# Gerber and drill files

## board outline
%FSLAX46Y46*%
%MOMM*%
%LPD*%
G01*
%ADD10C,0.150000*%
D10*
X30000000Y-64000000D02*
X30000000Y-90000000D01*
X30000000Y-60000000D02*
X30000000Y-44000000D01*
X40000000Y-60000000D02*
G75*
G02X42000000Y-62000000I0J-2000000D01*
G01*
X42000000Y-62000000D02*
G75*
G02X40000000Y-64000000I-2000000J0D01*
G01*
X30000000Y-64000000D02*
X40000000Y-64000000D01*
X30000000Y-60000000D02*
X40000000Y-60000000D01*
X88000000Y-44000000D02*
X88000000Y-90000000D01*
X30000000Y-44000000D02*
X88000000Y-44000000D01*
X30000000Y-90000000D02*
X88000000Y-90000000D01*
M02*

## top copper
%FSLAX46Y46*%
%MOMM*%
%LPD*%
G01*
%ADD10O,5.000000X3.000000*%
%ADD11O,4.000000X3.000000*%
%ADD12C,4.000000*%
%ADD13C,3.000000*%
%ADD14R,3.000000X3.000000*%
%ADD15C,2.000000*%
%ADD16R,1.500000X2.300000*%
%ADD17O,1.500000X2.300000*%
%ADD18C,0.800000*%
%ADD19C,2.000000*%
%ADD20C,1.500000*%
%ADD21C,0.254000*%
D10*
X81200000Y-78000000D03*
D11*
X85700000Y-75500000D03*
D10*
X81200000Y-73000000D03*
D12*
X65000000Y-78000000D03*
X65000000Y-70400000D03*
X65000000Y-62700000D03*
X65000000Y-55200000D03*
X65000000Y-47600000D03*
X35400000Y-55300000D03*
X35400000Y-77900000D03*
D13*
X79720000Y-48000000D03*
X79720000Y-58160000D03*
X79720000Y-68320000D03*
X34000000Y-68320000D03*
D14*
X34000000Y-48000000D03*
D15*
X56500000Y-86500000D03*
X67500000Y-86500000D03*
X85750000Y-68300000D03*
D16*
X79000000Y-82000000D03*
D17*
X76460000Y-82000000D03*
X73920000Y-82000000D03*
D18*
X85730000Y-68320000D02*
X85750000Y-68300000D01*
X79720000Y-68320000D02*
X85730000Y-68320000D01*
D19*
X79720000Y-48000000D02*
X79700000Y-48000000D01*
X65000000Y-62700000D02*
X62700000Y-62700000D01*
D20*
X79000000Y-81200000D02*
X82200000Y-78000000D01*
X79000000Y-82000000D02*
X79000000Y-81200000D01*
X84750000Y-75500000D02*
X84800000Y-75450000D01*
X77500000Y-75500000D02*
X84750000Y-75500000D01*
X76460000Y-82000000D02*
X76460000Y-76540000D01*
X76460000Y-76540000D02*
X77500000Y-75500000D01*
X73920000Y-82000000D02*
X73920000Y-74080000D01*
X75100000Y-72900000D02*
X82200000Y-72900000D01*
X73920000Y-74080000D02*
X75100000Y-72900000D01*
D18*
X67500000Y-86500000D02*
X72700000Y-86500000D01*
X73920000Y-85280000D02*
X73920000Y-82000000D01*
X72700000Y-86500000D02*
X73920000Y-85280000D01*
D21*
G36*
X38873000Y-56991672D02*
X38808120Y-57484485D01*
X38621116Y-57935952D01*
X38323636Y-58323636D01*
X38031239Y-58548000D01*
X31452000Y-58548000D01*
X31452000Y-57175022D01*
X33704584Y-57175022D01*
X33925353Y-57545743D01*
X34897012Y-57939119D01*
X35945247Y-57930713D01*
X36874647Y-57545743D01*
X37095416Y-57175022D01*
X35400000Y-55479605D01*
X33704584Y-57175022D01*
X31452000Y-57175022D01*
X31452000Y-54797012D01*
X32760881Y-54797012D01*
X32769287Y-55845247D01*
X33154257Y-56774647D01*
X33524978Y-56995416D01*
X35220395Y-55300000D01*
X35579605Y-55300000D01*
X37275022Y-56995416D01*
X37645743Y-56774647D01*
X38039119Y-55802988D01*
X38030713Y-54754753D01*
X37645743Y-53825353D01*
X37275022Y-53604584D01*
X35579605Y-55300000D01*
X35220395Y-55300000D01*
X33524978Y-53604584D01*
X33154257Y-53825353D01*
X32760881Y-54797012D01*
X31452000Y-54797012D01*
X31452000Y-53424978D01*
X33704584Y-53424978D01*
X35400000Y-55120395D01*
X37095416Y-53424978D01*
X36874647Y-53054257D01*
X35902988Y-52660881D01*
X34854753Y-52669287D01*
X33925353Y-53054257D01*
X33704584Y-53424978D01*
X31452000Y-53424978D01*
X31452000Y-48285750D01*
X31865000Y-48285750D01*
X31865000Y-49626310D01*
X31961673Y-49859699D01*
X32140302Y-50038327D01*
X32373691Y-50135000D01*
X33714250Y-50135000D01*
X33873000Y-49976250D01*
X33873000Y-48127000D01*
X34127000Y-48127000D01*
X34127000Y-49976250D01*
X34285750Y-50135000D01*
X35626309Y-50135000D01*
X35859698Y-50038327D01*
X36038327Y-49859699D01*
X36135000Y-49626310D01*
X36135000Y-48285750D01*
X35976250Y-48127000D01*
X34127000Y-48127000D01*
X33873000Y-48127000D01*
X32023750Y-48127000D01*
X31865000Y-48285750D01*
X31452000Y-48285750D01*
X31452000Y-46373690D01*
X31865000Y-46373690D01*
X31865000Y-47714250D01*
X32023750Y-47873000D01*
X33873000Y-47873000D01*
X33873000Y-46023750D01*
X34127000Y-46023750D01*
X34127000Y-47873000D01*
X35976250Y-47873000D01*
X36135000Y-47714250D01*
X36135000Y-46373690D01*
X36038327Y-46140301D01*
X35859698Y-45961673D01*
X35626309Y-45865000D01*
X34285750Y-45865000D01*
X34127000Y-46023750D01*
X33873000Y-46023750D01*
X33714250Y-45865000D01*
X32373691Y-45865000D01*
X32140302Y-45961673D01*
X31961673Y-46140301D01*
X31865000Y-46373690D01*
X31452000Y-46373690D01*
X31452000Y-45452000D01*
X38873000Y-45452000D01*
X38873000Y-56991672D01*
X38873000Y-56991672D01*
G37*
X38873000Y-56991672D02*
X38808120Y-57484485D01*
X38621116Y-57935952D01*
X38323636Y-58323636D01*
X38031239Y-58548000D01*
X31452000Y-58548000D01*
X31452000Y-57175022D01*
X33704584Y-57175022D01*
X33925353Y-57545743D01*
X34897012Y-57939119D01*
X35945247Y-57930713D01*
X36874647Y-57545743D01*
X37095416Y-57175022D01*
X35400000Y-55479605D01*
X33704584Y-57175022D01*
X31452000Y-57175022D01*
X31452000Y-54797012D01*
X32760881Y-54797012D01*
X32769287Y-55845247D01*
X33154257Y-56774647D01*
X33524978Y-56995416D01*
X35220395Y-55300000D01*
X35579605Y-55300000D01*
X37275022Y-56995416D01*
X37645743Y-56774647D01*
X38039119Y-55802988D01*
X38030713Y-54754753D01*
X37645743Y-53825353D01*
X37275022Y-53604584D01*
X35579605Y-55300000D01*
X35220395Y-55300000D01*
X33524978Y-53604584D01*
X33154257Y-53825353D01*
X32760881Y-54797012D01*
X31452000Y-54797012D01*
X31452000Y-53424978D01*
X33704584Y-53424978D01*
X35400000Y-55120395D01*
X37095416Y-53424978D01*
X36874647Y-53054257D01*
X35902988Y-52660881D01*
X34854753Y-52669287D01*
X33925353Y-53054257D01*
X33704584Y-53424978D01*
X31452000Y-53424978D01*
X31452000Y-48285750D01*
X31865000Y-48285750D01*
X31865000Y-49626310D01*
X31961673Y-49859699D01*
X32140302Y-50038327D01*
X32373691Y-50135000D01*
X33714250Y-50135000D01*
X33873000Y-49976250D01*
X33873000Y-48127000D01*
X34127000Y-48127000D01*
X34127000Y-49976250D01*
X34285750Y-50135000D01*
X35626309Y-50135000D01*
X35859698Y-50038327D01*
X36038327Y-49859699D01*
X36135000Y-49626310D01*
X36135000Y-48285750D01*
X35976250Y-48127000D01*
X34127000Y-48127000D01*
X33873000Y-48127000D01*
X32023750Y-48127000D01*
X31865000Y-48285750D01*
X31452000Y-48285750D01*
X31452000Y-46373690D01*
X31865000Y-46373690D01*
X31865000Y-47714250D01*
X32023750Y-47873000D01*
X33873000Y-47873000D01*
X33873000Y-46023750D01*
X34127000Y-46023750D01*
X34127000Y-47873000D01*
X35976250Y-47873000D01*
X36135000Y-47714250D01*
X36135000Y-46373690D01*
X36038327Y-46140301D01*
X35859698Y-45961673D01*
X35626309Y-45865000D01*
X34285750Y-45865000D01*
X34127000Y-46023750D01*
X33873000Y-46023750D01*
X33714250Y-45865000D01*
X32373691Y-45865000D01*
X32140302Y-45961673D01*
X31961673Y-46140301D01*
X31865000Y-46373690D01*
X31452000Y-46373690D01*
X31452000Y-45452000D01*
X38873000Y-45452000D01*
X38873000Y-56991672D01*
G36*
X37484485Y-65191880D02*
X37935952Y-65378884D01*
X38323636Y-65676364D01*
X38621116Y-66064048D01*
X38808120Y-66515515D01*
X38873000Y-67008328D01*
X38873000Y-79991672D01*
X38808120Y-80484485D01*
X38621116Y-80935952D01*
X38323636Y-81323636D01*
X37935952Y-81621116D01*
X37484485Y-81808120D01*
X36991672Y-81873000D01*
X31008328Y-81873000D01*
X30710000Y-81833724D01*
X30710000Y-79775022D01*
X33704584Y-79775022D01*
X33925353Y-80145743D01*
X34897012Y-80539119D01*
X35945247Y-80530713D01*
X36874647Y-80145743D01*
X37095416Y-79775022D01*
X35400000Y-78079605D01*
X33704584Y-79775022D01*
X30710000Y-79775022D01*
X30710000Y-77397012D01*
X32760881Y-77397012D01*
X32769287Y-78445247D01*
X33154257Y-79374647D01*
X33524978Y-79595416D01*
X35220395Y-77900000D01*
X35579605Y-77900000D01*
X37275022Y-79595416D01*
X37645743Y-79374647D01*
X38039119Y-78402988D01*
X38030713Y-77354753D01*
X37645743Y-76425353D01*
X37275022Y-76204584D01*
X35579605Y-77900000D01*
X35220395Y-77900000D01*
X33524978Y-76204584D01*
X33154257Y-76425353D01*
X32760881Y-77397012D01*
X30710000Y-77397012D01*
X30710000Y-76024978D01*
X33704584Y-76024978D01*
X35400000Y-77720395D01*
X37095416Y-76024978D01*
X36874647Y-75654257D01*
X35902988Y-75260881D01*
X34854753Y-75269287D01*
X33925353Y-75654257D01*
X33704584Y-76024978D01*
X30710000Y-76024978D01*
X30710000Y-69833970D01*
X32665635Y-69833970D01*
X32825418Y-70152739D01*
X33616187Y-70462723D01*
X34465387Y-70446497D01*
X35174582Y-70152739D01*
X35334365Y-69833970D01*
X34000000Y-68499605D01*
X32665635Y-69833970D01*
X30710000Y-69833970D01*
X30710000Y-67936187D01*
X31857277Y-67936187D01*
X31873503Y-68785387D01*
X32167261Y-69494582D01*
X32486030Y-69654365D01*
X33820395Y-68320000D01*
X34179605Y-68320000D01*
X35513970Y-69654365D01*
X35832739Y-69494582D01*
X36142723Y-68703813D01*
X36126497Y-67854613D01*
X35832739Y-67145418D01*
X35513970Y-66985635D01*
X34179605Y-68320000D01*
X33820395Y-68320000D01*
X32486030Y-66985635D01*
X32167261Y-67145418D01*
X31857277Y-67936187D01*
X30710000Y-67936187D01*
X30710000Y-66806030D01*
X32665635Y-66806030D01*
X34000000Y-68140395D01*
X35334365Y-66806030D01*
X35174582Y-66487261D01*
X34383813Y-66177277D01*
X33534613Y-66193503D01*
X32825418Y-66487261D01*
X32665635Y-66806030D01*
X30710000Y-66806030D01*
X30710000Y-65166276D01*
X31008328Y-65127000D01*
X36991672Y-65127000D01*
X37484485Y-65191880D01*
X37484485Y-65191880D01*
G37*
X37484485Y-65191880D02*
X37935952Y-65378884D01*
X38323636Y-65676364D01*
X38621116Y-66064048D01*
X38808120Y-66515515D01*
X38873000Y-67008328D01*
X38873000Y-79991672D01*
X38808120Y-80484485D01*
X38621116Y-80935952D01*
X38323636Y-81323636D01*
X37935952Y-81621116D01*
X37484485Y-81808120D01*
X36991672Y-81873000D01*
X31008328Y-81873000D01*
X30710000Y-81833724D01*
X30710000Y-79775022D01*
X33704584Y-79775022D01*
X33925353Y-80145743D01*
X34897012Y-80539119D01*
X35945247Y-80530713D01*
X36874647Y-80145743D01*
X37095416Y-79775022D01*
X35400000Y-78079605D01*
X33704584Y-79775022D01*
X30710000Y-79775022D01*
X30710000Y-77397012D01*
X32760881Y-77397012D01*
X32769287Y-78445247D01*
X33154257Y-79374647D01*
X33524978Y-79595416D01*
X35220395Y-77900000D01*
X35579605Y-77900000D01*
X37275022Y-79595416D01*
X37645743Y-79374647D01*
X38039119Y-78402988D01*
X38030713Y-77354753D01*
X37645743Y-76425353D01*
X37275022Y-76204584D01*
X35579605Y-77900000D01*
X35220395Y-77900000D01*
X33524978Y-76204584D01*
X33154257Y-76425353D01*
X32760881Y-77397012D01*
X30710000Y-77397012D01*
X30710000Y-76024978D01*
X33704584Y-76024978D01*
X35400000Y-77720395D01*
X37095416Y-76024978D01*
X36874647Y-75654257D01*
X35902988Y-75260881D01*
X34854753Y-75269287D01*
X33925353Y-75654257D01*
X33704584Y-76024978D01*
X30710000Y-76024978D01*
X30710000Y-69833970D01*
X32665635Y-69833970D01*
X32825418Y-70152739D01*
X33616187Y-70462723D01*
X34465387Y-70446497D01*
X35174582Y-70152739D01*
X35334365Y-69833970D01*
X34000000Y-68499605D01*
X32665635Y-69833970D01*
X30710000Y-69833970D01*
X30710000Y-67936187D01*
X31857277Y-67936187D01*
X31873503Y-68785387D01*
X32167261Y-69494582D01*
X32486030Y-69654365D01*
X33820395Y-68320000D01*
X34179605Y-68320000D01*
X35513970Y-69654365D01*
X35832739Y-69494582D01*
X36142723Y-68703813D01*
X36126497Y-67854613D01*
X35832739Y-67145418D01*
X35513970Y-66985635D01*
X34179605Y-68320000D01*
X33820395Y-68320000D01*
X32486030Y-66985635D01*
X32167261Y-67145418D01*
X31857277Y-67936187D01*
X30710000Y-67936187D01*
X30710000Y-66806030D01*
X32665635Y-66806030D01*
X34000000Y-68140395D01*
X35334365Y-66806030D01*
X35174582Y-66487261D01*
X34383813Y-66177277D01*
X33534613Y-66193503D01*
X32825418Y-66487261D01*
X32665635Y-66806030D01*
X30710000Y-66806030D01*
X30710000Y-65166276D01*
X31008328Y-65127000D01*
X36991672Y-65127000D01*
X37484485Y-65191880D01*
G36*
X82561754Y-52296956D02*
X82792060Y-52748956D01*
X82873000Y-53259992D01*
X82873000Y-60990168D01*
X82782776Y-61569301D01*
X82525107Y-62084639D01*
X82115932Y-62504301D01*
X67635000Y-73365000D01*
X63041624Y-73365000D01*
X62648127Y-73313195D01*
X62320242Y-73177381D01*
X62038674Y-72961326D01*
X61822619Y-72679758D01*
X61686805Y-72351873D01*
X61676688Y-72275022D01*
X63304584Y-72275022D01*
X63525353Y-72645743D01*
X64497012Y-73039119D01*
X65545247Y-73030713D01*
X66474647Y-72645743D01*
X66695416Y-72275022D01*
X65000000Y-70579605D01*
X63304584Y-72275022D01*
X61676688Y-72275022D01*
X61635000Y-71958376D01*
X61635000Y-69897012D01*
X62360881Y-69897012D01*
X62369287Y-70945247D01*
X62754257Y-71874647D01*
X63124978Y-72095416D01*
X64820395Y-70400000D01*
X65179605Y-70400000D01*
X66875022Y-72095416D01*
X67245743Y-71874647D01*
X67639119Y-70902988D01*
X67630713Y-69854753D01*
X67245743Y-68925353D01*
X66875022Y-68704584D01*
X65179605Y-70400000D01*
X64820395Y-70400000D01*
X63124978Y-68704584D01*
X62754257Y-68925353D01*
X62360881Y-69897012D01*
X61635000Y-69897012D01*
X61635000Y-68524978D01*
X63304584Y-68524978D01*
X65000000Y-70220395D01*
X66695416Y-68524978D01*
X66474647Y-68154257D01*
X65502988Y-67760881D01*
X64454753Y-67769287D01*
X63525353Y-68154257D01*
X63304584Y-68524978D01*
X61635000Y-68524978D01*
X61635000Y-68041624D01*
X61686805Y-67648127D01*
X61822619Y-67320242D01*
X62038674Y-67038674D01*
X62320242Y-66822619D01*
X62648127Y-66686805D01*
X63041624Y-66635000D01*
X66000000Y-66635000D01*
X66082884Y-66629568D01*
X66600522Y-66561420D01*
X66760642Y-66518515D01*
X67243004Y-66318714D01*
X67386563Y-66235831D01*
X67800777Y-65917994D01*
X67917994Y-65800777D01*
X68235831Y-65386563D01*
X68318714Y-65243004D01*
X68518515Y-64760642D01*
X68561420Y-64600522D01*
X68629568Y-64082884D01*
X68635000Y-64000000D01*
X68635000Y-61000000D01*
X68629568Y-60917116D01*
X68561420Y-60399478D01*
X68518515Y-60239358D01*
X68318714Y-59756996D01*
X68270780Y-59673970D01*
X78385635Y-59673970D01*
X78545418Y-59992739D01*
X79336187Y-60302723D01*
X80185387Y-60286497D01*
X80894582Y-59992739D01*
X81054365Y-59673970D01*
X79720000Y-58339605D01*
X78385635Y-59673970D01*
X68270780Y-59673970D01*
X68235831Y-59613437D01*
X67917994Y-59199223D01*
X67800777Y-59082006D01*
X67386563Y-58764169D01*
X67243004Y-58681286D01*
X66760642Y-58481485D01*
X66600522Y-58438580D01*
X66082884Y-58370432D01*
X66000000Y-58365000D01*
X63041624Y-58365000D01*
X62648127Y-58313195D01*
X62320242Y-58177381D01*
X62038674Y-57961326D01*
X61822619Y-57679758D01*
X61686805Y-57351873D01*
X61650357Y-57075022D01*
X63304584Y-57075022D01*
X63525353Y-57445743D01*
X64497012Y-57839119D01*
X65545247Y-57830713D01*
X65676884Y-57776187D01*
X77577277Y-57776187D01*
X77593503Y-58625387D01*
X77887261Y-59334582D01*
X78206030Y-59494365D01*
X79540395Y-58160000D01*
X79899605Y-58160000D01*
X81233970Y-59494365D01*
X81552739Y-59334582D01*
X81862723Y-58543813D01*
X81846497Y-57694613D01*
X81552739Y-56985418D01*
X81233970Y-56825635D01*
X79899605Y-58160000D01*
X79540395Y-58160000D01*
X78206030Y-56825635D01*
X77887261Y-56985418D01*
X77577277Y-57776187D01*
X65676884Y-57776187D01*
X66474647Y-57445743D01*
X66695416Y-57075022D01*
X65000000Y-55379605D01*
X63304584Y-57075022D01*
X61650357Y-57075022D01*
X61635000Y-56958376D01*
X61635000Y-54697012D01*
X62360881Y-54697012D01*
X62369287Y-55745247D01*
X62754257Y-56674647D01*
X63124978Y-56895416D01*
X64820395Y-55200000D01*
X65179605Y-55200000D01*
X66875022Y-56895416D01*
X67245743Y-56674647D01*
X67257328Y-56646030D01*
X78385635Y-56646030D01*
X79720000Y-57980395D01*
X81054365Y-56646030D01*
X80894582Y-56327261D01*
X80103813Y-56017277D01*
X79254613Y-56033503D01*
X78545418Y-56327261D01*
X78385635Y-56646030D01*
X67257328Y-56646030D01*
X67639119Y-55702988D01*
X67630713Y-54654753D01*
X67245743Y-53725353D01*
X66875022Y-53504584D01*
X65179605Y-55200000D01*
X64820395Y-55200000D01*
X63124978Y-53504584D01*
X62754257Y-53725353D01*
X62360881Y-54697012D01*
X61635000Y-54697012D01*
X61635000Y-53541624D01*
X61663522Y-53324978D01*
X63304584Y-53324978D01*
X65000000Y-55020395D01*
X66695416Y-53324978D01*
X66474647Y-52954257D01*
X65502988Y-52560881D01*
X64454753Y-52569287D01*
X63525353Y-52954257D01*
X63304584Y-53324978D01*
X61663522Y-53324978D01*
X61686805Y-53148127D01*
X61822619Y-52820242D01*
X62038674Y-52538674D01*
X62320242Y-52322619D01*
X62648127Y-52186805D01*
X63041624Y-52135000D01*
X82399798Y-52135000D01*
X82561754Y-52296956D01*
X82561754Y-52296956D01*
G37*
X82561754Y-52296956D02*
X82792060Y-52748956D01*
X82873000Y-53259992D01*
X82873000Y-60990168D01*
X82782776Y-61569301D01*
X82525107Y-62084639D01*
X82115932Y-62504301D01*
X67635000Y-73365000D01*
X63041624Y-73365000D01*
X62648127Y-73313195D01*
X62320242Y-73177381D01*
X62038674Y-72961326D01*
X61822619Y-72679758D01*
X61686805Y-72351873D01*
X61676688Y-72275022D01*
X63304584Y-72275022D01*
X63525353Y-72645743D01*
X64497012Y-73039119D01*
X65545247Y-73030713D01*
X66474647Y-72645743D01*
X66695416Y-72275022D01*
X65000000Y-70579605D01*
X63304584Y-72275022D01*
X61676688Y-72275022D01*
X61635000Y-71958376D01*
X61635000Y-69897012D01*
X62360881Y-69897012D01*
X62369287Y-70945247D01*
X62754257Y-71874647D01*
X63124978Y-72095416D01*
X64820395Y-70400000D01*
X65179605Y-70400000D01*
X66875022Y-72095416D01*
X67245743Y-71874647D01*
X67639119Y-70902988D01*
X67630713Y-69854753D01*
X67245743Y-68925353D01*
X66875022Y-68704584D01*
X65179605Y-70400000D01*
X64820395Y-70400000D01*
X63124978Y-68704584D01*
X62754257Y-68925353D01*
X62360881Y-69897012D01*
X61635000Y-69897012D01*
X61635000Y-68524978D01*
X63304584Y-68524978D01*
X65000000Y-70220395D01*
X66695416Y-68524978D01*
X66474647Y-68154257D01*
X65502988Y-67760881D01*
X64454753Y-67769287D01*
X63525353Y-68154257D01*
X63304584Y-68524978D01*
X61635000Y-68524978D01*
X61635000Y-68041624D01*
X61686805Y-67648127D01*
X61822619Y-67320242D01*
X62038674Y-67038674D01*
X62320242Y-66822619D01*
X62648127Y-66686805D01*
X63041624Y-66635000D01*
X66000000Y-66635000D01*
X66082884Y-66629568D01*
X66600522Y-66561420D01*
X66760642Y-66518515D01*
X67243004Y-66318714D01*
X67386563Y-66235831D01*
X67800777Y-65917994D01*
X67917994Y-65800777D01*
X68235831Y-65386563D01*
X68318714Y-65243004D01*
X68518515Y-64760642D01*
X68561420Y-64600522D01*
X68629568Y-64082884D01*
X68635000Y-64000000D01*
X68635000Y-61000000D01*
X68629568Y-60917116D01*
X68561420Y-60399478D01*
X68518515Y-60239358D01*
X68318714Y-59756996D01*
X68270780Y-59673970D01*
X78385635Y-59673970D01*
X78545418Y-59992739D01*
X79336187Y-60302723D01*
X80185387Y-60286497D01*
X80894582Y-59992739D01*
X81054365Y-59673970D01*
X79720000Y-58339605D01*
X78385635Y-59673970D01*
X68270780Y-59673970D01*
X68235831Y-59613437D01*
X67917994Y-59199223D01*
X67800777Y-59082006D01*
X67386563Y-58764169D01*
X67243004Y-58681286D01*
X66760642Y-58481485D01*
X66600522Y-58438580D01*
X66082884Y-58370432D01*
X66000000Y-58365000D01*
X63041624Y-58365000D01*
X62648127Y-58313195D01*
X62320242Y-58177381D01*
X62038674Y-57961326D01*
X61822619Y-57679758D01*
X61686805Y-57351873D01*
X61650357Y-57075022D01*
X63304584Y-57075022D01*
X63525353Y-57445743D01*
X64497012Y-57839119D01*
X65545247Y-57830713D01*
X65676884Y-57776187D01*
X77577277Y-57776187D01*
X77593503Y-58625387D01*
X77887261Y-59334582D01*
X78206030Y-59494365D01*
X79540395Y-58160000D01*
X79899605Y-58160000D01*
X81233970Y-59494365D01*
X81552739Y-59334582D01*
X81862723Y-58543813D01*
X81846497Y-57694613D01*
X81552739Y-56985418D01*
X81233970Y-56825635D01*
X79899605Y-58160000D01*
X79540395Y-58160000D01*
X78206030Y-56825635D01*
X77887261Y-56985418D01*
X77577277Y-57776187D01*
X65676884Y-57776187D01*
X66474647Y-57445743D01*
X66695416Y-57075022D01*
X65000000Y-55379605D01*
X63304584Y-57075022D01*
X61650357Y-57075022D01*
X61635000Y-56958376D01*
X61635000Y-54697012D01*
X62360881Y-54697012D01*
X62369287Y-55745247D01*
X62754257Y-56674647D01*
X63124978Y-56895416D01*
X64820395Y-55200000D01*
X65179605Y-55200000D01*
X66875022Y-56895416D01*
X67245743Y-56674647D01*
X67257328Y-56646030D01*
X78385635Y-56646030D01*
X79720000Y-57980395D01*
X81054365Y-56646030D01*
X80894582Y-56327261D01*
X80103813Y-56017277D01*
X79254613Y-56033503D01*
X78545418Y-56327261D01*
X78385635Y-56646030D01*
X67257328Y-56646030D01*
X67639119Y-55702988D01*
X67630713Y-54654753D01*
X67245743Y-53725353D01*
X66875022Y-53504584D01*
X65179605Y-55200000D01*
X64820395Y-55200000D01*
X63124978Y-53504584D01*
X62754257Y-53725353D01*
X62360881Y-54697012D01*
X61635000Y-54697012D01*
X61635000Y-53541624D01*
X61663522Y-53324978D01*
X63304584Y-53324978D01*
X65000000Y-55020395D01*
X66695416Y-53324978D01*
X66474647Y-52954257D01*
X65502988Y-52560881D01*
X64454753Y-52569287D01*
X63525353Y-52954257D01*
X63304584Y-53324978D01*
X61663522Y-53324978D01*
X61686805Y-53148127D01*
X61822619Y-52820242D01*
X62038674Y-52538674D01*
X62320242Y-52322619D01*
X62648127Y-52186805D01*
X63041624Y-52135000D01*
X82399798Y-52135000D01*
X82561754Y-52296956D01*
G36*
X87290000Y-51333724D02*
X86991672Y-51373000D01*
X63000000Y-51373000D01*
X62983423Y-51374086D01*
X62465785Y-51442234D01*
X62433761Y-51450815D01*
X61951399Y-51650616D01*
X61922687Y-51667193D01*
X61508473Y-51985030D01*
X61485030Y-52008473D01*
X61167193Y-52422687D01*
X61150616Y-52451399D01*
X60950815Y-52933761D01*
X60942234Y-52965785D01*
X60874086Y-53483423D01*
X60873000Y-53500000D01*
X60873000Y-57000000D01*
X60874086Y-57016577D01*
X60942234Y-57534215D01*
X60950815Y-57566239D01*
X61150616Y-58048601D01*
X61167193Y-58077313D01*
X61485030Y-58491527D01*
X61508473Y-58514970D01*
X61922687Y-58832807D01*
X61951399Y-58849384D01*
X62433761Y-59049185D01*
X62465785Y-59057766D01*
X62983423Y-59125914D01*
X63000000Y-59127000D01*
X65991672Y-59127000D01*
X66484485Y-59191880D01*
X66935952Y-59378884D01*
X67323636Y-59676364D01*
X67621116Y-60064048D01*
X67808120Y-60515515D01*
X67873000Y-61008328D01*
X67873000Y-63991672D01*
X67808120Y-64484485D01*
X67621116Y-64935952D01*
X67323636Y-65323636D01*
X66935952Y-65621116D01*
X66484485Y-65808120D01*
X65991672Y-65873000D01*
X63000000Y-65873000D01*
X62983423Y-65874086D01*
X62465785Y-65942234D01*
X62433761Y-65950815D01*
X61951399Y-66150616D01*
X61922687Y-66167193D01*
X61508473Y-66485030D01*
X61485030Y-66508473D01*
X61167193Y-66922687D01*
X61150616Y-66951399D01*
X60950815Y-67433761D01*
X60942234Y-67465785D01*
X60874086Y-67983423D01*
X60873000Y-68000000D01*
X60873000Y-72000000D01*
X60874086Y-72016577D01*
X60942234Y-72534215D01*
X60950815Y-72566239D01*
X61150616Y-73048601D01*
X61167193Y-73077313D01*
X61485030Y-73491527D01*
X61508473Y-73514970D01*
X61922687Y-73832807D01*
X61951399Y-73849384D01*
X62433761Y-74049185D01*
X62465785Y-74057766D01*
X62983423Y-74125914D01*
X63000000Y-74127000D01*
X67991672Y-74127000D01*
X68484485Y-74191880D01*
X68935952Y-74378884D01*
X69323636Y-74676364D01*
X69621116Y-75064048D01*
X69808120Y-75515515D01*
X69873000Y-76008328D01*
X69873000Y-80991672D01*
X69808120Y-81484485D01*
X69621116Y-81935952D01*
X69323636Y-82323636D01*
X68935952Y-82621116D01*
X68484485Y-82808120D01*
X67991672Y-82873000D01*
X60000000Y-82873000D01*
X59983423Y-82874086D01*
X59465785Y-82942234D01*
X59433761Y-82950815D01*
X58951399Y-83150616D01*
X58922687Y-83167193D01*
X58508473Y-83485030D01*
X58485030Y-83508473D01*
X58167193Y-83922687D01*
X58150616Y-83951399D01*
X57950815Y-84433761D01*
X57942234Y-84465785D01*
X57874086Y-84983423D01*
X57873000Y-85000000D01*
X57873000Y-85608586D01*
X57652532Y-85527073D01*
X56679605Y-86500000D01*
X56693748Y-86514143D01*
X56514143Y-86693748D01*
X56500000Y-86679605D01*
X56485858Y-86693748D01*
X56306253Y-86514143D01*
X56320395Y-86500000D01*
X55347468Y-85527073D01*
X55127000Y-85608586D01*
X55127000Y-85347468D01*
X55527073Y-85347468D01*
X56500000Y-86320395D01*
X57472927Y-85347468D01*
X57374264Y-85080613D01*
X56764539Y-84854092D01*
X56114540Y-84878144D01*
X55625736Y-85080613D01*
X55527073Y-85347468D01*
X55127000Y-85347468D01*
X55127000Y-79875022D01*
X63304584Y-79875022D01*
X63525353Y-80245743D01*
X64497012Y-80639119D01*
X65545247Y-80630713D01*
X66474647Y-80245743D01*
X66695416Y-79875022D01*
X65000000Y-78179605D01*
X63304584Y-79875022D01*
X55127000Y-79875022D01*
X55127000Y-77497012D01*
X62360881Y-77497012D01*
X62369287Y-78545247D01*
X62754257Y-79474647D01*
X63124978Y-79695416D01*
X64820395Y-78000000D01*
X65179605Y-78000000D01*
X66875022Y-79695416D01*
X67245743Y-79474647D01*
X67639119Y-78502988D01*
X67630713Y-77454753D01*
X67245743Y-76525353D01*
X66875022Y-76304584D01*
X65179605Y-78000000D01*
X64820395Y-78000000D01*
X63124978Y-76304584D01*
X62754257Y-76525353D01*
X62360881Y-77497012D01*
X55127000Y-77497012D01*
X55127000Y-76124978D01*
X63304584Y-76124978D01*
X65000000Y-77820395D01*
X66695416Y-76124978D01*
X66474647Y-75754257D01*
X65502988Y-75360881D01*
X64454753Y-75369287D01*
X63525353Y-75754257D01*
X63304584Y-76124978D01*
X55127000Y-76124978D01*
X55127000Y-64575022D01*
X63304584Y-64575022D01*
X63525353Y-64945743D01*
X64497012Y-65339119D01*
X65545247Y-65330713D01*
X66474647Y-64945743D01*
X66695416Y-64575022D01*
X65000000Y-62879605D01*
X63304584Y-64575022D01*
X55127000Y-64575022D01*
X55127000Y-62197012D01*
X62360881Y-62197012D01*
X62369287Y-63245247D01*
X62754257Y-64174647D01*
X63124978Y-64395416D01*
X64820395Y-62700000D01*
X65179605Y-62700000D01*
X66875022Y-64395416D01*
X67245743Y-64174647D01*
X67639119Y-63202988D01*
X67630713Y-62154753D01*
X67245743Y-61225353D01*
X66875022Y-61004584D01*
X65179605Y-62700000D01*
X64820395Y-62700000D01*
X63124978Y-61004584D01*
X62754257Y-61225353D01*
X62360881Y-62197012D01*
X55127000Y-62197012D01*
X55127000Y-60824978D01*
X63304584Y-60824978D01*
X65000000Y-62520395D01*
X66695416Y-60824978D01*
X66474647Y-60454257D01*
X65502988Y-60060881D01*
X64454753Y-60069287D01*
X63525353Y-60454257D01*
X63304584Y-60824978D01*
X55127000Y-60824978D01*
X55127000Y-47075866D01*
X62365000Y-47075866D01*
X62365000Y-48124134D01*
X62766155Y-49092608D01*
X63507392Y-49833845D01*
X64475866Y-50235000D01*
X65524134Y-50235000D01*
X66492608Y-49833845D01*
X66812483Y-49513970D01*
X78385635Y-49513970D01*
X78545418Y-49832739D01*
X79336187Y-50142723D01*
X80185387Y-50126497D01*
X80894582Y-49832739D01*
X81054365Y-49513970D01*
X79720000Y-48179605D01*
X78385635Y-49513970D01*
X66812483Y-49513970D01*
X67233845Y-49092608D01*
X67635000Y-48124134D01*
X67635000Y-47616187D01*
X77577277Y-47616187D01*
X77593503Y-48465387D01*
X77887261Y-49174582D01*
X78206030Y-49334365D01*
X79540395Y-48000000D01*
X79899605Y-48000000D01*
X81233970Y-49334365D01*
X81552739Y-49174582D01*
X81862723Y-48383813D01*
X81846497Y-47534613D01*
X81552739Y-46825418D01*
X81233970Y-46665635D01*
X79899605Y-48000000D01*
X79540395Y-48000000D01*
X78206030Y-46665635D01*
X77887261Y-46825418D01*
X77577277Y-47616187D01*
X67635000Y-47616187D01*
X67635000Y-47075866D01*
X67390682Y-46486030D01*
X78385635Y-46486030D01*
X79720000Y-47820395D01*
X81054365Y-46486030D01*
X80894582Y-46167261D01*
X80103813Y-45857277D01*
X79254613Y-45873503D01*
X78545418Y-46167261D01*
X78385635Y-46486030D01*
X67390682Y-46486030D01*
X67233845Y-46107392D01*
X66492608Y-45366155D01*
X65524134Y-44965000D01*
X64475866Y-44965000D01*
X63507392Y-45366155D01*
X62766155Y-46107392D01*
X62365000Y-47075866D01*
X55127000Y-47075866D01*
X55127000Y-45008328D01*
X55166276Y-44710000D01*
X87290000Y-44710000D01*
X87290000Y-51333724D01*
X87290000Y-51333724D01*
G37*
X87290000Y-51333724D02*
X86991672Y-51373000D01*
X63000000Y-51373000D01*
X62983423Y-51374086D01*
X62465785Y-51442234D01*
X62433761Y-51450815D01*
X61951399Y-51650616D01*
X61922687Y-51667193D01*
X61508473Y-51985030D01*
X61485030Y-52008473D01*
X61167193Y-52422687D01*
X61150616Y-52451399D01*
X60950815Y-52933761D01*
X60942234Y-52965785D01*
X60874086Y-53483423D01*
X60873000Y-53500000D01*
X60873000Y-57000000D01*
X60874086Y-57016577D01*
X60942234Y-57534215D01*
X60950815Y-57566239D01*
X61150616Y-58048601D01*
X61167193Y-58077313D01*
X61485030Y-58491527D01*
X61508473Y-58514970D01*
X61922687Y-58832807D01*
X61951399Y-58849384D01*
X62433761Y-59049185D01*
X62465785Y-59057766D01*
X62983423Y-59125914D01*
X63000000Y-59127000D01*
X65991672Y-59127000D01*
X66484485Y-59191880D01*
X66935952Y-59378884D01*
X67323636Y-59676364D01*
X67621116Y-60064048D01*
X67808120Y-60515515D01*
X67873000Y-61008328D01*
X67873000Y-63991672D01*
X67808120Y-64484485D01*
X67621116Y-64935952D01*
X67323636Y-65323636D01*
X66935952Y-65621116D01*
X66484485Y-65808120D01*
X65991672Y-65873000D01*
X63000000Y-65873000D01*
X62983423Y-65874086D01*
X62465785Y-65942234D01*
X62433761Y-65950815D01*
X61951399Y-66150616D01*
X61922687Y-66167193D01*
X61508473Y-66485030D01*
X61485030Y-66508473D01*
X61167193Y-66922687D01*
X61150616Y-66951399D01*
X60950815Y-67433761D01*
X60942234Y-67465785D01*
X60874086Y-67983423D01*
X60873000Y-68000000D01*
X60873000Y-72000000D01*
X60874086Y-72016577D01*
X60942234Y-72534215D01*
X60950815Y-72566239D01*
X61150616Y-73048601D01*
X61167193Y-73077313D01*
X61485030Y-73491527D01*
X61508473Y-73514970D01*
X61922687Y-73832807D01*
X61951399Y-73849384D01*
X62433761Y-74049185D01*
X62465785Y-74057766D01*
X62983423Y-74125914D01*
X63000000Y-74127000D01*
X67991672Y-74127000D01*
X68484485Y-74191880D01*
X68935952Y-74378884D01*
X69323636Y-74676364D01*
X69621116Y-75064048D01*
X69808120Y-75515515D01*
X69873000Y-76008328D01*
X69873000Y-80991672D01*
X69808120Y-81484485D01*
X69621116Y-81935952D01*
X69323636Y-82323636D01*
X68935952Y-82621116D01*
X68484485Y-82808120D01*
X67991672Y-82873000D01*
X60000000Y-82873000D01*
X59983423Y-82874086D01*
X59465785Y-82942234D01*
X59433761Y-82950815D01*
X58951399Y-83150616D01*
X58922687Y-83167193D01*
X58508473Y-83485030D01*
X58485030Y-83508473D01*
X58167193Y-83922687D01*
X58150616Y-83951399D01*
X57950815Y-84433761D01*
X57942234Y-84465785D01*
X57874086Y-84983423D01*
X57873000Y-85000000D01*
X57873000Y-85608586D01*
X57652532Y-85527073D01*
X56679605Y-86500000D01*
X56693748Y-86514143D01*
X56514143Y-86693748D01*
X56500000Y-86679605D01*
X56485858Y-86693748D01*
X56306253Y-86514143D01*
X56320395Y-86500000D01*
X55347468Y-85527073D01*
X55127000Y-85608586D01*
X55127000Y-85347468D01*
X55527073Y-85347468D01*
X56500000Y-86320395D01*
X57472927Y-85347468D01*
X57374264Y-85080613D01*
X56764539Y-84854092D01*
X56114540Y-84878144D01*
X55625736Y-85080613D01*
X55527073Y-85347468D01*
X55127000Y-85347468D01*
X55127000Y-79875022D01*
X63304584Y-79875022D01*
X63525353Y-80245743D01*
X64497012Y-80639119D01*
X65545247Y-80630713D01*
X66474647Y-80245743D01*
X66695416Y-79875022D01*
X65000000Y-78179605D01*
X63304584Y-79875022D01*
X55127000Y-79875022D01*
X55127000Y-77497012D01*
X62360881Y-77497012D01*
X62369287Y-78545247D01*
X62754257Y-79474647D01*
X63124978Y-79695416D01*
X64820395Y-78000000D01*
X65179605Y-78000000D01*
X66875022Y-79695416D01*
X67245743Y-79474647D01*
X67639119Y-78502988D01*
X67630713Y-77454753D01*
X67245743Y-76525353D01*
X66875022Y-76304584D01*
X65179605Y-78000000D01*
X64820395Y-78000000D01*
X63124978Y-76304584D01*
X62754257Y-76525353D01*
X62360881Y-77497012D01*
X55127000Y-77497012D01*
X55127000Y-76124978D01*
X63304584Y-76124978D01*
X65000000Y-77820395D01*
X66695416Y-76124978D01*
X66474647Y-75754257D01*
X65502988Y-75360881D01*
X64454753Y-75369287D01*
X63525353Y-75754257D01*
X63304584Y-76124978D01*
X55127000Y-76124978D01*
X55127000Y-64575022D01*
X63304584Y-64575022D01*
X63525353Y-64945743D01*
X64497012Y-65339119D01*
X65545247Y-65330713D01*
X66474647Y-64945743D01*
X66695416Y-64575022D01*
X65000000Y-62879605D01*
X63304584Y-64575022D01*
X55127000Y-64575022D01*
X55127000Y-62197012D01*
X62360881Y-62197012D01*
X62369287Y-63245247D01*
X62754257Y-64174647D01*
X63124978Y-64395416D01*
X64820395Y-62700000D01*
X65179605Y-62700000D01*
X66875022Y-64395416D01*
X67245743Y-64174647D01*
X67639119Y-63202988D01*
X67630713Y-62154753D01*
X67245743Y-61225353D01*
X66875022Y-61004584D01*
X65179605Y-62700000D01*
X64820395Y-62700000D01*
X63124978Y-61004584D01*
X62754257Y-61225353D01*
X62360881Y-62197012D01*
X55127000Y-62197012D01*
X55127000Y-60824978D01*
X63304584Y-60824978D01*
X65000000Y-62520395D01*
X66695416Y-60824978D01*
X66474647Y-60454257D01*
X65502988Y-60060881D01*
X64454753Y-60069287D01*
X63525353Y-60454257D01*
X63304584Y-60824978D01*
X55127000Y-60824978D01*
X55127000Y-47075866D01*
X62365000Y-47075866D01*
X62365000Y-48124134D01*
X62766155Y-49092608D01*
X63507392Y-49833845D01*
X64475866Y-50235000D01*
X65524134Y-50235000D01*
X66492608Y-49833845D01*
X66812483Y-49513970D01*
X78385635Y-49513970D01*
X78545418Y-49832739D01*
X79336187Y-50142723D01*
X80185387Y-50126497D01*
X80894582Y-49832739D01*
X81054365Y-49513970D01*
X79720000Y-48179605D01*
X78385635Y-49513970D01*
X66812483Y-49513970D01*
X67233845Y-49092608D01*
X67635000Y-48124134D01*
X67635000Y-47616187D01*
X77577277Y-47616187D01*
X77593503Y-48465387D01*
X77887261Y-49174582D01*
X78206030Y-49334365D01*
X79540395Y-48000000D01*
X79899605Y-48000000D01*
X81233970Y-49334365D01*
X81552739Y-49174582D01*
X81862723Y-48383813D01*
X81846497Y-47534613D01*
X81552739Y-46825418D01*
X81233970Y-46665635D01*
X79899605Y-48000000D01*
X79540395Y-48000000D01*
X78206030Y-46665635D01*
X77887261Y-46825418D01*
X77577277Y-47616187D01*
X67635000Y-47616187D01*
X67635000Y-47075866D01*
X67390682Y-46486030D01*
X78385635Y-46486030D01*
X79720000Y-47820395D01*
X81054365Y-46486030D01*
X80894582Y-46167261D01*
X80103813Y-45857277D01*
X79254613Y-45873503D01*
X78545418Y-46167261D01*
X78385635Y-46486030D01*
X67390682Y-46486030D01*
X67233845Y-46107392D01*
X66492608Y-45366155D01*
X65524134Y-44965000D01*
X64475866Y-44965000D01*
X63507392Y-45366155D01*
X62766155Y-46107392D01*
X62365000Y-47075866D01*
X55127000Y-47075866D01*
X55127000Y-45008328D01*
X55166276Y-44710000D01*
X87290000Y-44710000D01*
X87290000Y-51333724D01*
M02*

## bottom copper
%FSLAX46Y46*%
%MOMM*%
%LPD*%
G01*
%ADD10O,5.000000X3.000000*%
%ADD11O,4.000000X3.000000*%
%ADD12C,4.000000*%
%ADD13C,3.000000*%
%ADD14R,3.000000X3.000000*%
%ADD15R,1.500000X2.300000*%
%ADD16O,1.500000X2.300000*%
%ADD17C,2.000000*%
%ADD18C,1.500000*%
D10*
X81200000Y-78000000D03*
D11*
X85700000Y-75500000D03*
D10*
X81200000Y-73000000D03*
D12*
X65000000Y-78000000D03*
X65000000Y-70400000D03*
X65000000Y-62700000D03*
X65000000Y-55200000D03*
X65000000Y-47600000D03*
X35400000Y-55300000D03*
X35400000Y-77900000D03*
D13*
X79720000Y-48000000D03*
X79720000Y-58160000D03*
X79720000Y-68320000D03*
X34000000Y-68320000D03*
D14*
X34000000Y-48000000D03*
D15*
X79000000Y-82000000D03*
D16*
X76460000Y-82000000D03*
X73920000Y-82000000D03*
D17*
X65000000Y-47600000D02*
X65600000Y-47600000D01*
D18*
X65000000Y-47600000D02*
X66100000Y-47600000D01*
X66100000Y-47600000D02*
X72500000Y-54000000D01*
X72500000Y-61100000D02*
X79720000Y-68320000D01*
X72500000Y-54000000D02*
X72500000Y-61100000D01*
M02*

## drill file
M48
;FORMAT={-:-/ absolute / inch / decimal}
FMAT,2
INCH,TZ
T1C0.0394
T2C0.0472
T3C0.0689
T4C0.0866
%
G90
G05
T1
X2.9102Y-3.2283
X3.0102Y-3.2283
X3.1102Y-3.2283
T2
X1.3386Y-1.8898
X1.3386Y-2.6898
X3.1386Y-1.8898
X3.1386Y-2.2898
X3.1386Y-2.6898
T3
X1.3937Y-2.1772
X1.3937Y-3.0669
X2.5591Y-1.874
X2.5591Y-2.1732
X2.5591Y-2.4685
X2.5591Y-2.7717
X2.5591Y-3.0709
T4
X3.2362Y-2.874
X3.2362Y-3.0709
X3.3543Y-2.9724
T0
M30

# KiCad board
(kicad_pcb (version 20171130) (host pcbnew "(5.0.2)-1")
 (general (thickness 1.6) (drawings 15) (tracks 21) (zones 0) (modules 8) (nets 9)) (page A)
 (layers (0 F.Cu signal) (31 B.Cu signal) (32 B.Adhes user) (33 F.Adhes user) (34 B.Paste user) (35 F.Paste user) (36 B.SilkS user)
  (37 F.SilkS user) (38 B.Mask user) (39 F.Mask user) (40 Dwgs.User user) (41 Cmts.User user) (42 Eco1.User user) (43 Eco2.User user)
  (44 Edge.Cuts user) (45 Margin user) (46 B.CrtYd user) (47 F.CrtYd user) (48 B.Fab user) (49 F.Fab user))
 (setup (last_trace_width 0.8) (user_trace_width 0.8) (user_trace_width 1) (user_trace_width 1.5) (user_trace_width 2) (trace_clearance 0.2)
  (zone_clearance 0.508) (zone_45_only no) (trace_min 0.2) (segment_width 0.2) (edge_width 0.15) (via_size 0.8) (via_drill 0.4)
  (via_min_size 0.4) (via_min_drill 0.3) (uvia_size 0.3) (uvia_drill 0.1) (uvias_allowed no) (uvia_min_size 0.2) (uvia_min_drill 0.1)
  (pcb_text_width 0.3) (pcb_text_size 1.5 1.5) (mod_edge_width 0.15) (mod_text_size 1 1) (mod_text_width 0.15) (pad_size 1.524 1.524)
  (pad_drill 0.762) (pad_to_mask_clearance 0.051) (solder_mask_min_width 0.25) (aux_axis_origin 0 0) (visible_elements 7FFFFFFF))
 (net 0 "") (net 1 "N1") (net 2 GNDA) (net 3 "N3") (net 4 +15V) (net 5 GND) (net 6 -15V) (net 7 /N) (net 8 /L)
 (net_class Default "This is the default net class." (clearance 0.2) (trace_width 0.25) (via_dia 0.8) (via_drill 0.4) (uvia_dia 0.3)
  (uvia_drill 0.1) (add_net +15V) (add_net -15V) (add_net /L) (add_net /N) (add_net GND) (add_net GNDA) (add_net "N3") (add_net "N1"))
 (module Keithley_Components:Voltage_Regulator (layer F.Cu) (at 82.2 78 270)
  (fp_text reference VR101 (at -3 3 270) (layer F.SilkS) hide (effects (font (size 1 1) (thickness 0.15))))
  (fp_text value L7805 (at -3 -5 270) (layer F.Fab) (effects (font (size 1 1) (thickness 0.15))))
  (pad 1 thru_hole oval (at 0 0 270) (size 3 5) (drill 2.2 (offset 0 1)) (layers *.Cu *.Mask) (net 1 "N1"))
  (pad 2 thru_hole oval (at -2.5 -3 270) (size 3 4) (drill 2.2 (offset 0 -0.5)) (layers *.Cu *.Mask) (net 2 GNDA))
  (pad 3 thru_hole oval (at -5 0 270) (size 3 5) (drill 2.2 (offset 0 1)) (layers *.Cu *.Mask) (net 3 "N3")))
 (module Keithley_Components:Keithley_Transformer (layer F.Cu) (at 65 83 180)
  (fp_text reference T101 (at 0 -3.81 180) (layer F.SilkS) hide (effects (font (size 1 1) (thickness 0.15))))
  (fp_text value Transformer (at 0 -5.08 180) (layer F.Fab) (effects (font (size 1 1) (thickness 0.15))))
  (pad 2 thru_hole circle (at 0 5 180) (size 4 4) (drill 1.75) (layers *.Cu *.Mask) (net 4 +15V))
  (pad 3 thru_hole circle (at 0 12.6 180) (size 4 4) (drill 1.75) (layers *.Cu *.Mask) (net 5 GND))
  (pad 4 thru_hole circle (at 0 20.3 180) (size 4 4) (drill 1.75) (layers *.Cu *.Mask) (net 4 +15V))
  (pad 5 thru_hole circle (at 0 27.8 180) (size 4 4) (drill 1.75) (layers *.Cu *.Mask) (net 5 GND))
  (pad 6 thru_hole circle (at 0 35.4 180) (size 4 4) (drill 1.75) (layers *.Cu *.Mask) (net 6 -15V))
  (pad 8 thru_hole circle (at 29.6 27.7 180) (size 4 4) (drill 1.75) (layers *.Cu *.Mask) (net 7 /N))
  (pad 11 thru_hole circle (at 29.6 5.1 180) (size 4 4) (drill 1.75) (layers *.Cu *.Mask) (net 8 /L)))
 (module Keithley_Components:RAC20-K (layer F.Cu) (at 34 48)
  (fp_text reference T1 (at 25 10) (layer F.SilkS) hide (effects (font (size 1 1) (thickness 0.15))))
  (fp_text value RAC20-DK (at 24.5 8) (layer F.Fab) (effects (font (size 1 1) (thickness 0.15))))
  (pad 5 thru_hole circle (at 45.72 0) (size 3 3) (drill 1.2) (layers *.Cu *.Mask) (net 4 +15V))
  (pad 4 thru_hole circle (at 45.72 10.16) (size 3 3) (drill 1.2) (layers *.Cu *.Mask) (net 5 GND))
  (pad 3 thru_hole circle (at 45.72 20.32) (size 3 3) (drill 1.2) (layers *.Cu *.Mask) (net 6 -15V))
  (pad 2 thru_hole circle (at 0 20.32) (size 3 3) (drill 1.2) (layers *.Cu *.Mask) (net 8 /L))
  (pad 1 thru_hole rect (at 0 0) (size 3 3) (drill 1.2) (layers *.Cu *.Mask) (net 7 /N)))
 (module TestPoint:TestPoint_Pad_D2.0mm (layer F.Cu) (at 56.5 86.5)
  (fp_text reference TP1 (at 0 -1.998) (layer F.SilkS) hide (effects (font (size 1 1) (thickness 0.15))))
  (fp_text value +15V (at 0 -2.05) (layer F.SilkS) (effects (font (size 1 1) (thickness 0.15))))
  (pad 1 smd circle (at 0 0) (size 2 2) (layers F.Cu F.Mask) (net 4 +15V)))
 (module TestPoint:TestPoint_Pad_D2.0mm (layer F.Cu) (at 67.5 86.5)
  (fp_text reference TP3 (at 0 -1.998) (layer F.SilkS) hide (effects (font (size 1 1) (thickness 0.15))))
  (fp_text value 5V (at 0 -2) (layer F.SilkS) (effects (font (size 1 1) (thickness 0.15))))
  (pad 1 smd circle (at 0 0) (size 2 2) (layers F.Cu F.Mask) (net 3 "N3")))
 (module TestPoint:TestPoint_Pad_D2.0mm (layer F.Cu) (at 85.75 68.3)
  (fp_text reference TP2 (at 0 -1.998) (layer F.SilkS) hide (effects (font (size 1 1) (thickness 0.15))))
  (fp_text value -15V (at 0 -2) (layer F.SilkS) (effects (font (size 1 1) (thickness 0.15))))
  (pad 1 smd circle (at 0 0) (size 2 2) (layers F.Cu F.Mask) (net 6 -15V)))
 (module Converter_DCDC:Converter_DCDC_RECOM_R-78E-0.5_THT (layer F.Cu) (at 79 82 180)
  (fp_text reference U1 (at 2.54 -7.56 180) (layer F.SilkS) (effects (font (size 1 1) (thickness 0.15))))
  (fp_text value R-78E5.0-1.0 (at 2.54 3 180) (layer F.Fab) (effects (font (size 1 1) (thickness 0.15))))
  (pad 1 thru_hole rect (at 0 0 180) (size 1.5 2.3) (drill 1) (layers *.Cu *.Mask) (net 1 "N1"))
  (pad 2 thru_hole oval (at 2.54 0 180) (size 1.5 2.3) (drill 1) (layers *.Cu *.Mask) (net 2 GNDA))
  (pad 3 thru_hole oval (at 5.08 0 180) (size 1.5 2.3) (drill 1) (layers *.Cu *.Mask) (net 3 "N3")))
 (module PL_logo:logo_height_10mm (layer F.Cu) (at 43.75 80)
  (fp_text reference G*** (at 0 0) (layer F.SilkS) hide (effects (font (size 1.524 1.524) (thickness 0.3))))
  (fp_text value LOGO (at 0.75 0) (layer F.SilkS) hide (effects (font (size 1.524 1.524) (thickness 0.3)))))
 (gr_line (start 30 64) (end 30 90) (layer Edge.Cuts) (width 0.15))
 (gr_line (start 30 60) (end 30 44) (layer Edge.Cuts) (width 0.15))
 (gr_arc (start 40 62) (end 42 62) (angle -90) (layer Edge.Cuts) (width 0.15))
 (gr_arc (start 40 62) (end 40 64) (angle -90) (layer Edge.Cuts) (width 0.15))
 (gr_line (start 30 64) (end 40 64) (layer Edge.Cuts) (width 0.15))
 (gr_line (start 30 60) (end 40 60) (layer Edge.Cuts) (width 0.15))
 (gr_line (start 88 44) (end 88 90) (layer Edge.Cuts) (width 0.15))
 (gr_line (start 30 44) (end 88 44) (layer Edge.Cuts) (width 0.15))
 (gr_line (start 30 90) (end 88 90) (layer Edge.Cuts) (width 0.15))
 (segment (start 65 47.6) (end 65.6 47.6) (width 2) (layer B.Cu) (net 6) (status 30))
 (segment (start 65 47.6) (end 66.1 47.6) (width 1.5) (layer B.Cu) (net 6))
 (segment (start 66.1 47.6) (end 72.5 54) (width 1.5) (layer B.Cu) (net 6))
 (segment (start 72.5 61.1) (end 79.72 68.32) (width 1.5) (layer B.Cu) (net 6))
 (segment (start 72.5 54) (end 72.5 61.1) (width 1.5) (layer B.Cu) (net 6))
 (segment (start 85.73 68.32) (end 85.75 68.3) (width 0.8) (layer F.Cu) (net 6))
 (segment (start 79.72 68.32) (end 85.73 68.32) (width 0.8) (layer F.Cu) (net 6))
 (segment (start 79.72 48) (end 79.7 48) (width 2) (layer F.Cu) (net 4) (status 30))
 (segment (start 65 62.7) (end 62.7 62.7) (width 2) (layer F.Cu) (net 4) (status 10))
 (segment (start 79 81.2) (end 82.2 78) (width 1.5) (layer F.Cu) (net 1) (status 30))
 (segment (start 79 82) (end 79 81.2) (width 1.5) (layer F.Cu) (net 1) (status 30))
 (segment (start 84.75 75.5) (end 84.8 75.45) (width 1.5) (layer F.Cu) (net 2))
 (segment (start 77.5 75.5) (end 84.75 75.5) (width 1.5) (layer F.Cu) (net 2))
 (segment (start 76.46 82) (end 76.46 76.54) (width 1.5) (layer F.Cu) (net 2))
 (segment (start 76.46 76.54) (end 77.5 75.5) (width 1.5) (layer F.Cu) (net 2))
 (segment (start 73.92 82) (end 73.92 74.08) (width 1.5) (layer F.Cu) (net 3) (status 10))
 (segment (start 75.1 72.9) (end 82.2 72.9) (width 1.5) (layer F.Cu) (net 3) (status 20))
 (segment (start 73.92 74.08) (end 75.1 72.9) (width 1.5) (layer F.Cu) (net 3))
 (segment (start 67.5 86.5) (end 72.7 86.5) (width 0.8) (layer F.Cu) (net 3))
 (segment (start 73.92 85.28) (end 73.92 82) (width 0.8) (layer F.Cu) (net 3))
 (segment (start 72.7 86.5) (end 73.92 85.28) (width 0.8) (layer F.Cu) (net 3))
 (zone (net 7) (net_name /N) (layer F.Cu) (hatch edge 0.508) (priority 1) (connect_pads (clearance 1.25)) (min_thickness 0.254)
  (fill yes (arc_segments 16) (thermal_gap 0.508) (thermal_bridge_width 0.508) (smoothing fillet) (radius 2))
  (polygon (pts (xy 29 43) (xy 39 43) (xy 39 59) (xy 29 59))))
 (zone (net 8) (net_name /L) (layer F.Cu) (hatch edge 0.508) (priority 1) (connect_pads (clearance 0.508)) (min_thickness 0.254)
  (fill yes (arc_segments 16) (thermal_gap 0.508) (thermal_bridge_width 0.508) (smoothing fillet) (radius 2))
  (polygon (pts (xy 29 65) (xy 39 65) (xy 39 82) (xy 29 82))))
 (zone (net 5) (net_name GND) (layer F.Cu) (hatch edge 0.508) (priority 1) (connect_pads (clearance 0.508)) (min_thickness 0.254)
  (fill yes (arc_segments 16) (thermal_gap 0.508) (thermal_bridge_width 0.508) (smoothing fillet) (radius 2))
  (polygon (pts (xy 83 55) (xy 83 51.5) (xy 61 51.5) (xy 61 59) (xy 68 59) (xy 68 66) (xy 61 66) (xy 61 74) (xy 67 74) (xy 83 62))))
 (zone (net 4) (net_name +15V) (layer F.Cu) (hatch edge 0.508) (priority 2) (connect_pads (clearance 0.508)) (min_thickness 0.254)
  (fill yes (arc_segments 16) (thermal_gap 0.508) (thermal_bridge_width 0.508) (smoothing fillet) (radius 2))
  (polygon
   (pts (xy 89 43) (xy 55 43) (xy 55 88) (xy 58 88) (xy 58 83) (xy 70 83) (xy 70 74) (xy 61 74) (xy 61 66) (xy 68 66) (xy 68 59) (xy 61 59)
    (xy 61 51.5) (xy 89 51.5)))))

